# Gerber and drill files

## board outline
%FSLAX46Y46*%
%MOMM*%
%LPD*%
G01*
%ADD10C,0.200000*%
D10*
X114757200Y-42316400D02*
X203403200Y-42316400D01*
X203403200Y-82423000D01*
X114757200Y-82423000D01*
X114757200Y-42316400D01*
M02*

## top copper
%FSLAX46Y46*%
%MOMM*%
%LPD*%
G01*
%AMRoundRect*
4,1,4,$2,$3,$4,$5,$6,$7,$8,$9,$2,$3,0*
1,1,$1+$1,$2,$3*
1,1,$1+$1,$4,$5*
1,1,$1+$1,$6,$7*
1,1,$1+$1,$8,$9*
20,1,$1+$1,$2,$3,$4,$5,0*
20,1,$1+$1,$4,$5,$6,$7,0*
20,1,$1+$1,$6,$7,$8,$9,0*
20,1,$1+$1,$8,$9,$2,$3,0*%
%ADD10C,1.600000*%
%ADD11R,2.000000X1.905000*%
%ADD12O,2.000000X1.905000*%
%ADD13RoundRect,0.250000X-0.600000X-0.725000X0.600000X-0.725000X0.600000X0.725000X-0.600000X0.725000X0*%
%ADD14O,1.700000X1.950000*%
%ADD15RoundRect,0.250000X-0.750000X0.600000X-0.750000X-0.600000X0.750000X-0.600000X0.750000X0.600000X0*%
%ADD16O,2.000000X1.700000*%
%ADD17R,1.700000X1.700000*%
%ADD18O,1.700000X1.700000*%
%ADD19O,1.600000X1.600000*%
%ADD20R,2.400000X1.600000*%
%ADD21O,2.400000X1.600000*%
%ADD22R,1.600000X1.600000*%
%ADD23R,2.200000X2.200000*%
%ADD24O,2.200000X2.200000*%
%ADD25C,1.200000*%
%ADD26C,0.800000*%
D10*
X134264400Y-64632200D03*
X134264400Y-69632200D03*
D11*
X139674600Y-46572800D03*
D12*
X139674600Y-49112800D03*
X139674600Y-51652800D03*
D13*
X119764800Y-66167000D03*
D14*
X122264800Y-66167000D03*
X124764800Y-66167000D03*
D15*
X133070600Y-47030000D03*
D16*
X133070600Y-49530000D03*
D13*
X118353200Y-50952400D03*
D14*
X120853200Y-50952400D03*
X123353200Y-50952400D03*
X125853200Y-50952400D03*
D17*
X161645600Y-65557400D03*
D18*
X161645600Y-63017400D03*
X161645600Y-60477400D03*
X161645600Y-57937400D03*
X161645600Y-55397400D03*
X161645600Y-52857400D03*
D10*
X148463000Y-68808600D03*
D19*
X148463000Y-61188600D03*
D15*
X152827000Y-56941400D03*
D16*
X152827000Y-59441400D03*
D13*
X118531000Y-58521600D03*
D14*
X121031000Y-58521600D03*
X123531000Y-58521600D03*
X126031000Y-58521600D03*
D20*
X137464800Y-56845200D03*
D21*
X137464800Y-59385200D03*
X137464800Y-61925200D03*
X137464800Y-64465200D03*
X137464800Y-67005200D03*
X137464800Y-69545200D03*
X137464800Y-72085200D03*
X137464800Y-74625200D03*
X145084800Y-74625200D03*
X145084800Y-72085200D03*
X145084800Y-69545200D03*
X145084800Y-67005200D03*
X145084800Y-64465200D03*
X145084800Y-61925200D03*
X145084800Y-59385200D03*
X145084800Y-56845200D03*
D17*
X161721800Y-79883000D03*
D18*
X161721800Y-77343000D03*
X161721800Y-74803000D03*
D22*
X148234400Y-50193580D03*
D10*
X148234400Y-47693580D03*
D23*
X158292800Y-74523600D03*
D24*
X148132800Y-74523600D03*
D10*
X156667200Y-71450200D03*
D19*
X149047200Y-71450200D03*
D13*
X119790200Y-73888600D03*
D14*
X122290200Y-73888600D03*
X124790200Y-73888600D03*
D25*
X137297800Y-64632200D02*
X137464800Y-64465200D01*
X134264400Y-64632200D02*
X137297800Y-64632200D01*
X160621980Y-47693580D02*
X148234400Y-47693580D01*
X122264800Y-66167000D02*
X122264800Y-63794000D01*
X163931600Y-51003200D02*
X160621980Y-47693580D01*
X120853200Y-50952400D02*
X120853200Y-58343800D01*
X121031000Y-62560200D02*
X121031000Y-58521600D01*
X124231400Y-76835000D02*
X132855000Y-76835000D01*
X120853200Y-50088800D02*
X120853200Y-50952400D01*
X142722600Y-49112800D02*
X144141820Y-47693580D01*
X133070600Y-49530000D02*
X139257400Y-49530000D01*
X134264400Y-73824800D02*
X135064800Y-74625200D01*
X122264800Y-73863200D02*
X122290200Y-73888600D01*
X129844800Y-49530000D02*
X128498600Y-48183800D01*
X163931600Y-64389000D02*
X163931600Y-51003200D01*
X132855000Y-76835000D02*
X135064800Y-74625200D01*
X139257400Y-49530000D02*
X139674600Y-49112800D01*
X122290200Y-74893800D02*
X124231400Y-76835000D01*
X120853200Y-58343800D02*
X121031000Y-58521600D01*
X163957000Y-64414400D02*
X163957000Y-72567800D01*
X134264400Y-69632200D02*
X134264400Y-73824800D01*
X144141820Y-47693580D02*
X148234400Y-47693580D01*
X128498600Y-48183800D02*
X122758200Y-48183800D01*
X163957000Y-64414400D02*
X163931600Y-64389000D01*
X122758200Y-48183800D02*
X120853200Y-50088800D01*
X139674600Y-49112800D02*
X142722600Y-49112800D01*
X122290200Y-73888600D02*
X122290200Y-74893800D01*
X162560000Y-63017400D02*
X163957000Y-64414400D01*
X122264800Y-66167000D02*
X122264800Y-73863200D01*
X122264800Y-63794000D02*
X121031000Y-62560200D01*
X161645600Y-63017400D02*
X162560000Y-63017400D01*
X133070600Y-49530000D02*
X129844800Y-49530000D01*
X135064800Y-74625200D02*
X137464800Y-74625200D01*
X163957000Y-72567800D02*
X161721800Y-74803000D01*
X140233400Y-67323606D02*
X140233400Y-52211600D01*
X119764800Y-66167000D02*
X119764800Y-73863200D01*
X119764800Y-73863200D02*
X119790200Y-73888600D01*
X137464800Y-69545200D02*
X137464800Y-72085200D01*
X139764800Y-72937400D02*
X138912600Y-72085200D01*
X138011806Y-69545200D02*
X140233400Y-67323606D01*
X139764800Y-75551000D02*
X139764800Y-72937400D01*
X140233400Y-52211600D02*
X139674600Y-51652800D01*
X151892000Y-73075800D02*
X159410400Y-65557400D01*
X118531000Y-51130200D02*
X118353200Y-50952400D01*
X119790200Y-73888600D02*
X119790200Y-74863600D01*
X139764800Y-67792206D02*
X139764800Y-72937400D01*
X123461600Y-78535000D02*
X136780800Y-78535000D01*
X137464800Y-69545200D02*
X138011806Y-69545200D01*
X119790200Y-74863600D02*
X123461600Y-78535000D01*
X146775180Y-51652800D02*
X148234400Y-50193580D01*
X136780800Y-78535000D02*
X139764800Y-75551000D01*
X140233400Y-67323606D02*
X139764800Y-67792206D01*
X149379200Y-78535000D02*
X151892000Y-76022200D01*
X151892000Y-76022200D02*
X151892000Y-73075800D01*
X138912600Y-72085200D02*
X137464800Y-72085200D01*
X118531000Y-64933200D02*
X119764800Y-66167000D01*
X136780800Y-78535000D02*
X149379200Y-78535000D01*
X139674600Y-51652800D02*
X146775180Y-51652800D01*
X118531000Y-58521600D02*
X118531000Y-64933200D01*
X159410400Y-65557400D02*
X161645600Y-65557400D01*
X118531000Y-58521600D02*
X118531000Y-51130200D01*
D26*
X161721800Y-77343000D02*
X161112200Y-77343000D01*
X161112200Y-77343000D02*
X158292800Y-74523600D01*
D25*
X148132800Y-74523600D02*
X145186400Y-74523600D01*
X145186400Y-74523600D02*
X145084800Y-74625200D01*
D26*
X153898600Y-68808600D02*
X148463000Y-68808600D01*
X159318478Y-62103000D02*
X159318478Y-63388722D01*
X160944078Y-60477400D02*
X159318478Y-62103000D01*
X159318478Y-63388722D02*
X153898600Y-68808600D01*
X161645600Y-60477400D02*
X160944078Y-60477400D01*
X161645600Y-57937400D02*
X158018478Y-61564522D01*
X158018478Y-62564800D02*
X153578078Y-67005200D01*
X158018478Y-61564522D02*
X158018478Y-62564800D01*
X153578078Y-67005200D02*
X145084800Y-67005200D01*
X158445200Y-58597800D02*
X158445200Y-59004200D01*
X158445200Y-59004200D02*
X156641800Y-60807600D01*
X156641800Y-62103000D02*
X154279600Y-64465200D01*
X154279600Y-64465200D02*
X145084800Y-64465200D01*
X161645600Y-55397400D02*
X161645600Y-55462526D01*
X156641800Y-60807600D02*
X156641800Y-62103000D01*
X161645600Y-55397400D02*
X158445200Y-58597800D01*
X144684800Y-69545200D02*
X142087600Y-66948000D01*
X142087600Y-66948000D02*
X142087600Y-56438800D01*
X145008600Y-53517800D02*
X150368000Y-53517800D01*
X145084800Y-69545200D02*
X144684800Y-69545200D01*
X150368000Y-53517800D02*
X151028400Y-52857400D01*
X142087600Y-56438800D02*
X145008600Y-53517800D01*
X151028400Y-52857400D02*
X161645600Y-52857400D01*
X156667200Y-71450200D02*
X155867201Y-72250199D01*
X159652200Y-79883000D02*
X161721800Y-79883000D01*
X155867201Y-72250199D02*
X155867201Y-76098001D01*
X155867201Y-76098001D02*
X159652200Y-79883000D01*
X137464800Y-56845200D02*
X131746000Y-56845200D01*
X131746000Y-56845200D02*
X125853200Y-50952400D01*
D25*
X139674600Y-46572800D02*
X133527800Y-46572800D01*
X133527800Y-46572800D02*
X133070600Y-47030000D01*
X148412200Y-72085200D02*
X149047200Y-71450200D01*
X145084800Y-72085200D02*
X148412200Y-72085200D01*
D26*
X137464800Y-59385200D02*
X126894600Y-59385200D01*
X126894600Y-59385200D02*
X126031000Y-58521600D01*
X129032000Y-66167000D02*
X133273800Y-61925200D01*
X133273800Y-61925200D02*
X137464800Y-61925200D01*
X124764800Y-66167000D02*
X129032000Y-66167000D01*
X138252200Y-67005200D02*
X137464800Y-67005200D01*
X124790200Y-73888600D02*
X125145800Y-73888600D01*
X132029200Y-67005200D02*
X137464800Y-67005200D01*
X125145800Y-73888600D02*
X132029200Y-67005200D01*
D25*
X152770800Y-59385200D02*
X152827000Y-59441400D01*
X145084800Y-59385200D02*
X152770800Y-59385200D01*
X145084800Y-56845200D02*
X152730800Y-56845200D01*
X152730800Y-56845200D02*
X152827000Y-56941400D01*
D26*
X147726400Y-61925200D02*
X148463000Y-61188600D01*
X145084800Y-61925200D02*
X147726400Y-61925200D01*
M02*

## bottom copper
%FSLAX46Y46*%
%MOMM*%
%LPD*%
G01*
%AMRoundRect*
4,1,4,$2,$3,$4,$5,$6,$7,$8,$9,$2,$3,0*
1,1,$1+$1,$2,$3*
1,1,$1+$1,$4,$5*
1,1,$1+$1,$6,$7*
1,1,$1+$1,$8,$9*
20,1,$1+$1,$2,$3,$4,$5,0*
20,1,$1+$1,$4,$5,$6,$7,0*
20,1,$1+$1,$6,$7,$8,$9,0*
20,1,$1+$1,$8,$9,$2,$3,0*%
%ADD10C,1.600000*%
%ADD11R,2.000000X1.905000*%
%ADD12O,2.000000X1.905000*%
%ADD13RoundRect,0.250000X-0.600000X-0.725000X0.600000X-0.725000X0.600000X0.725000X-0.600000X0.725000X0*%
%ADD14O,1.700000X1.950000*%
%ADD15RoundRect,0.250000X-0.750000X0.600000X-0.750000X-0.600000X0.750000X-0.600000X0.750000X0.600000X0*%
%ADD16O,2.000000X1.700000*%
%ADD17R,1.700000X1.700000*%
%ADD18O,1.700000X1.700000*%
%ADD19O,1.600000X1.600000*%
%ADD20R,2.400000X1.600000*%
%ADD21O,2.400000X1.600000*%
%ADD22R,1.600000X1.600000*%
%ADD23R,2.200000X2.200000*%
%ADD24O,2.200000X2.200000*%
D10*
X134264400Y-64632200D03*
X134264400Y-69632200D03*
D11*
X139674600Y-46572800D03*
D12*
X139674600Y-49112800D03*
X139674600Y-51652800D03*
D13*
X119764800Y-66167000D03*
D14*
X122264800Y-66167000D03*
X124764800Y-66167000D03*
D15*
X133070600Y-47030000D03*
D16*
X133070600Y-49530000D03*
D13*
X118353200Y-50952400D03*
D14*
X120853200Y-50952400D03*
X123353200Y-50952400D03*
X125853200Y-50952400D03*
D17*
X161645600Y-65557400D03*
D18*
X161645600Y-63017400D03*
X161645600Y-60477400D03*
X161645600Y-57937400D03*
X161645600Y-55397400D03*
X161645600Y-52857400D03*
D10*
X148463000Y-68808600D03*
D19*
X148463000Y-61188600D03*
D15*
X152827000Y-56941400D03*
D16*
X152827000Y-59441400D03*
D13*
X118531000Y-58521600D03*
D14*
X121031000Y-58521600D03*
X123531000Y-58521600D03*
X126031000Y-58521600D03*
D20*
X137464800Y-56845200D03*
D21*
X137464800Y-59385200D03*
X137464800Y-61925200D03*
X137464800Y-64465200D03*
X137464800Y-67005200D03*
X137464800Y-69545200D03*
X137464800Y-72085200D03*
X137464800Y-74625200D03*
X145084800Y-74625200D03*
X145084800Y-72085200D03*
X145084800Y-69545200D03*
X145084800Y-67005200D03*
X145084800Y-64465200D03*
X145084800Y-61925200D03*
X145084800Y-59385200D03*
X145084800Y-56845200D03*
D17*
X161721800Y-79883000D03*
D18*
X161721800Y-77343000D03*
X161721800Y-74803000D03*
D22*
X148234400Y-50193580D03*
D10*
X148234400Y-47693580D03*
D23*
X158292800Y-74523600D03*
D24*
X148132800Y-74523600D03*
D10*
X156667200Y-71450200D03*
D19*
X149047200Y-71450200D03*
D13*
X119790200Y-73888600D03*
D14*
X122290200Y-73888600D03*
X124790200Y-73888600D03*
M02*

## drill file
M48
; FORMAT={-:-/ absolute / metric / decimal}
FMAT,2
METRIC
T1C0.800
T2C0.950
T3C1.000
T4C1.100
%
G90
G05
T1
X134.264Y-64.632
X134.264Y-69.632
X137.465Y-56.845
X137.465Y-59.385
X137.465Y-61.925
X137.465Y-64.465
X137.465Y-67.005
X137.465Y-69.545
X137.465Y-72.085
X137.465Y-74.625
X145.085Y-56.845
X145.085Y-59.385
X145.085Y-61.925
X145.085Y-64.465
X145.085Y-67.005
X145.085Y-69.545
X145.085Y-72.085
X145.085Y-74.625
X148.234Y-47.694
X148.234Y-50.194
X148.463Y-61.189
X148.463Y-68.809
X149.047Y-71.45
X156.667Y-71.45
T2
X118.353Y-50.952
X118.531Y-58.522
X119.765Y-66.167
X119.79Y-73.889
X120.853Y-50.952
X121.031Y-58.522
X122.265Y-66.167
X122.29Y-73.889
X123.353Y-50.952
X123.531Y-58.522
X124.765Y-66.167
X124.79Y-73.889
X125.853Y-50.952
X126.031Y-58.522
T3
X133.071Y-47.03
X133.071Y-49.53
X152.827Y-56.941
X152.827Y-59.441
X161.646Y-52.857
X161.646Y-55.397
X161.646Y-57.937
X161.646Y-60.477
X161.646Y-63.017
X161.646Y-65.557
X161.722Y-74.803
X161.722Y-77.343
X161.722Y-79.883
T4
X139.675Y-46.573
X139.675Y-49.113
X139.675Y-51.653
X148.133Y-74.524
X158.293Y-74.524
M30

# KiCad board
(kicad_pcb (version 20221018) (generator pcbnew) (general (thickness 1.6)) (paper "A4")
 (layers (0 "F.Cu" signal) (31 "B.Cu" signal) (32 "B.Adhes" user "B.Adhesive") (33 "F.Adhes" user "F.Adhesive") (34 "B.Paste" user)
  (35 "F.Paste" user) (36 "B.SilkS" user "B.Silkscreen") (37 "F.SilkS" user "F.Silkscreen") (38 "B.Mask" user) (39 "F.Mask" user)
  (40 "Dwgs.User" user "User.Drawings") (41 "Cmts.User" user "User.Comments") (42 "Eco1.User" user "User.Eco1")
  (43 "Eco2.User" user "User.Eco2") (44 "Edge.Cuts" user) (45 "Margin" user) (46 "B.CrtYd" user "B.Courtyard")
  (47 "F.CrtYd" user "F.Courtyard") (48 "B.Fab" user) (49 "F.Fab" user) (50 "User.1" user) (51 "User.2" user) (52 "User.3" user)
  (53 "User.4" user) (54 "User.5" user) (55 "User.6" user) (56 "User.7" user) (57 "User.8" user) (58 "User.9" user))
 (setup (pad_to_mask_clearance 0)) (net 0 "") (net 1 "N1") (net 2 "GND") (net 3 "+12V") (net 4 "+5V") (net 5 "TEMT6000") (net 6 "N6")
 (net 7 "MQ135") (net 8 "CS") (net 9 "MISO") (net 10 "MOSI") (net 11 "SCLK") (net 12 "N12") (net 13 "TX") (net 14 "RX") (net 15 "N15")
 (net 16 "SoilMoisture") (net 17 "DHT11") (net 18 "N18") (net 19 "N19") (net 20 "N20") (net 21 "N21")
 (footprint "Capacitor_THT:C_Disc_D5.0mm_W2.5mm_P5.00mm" (layer "F.Cu") (at 134.2644 64.6322 -90)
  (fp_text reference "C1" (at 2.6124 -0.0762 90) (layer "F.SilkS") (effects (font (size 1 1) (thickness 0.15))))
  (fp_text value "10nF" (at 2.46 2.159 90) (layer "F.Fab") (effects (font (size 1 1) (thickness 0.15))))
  (pad "1" thru_hole circle (at 0 0 270) (size 1.6 1.6) (drill 0.8) (layers "*.Cu" "*.Mask") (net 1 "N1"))
  (pad "2" thru_hole circle (at 5 0 270) (size 1.6 1.6) (drill 0.8) (layers "*.Cu" "*.Mask") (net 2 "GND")))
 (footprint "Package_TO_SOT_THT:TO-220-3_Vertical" (layer "F.Cu") (at 139.6746 46.5728 -90)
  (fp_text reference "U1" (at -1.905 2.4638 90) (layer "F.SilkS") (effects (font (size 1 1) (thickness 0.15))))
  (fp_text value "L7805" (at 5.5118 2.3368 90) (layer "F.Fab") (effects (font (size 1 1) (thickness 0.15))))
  (pad "1" thru_hole rect (at 0 0 270) (size 1.905 2) (drill 1.1) (layers "*.Cu" "*.Mask") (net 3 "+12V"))
  (pad "2" thru_hole oval (at 2.54 0 270) (size 1.905 2) (drill 1.1) (layers "*.Cu" "*.Mask") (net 2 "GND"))
  (pad "3" thru_hole oval (at 5.08 0 270) (size 1.905 2) (drill 1.1) (layers "*.Cu" "*.Mask") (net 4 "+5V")))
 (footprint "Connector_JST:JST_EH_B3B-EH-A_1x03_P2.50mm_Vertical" (layer "F.Cu") (at 119.7648 66.167)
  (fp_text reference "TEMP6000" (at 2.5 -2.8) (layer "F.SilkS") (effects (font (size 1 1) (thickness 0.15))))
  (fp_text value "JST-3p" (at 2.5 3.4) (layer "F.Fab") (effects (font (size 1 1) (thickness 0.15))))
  (pad "1" thru_hole roundrect (at 0 0) (size 1.7 1.95) (drill 0.95) (layers "*.Cu" "*.Mask") (roundrect_rratio 0.147059) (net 4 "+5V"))
  (pad "2" thru_hole oval (at 2.5 0) (size 1.7 1.95) (drill 0.95) (layers "*.Cu" "*.Mask") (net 2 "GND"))
  (pad "3" thru_hole oval (at 5 0) (size 1.7 1.95) (drill 0.95) (layers "*.Cu" "*.Mask") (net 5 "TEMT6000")))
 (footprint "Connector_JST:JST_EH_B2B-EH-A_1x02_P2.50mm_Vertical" (layer "F.Cu") (at 133.0706 47.03 -90)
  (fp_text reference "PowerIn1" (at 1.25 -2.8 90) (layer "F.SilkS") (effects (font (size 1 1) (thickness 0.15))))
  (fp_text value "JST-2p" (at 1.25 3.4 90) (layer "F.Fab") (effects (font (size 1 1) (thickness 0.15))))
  (pad "1" thru_hole roundrect (at 0 0 270) (size 1.7 2) (drill 1) (layers "*.Cu" "*.Mask") (roundrect_rratio 0.147059) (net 3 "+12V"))
  (pad "2" thru_hole oval (at 2.5 0 270) (size 1.7 2) (drill 1) (layers "*.Cu" "*.Mask") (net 2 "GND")))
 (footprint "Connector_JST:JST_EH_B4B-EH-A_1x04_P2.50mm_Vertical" (layer "F.Cu") (at 118.3532 50.9524)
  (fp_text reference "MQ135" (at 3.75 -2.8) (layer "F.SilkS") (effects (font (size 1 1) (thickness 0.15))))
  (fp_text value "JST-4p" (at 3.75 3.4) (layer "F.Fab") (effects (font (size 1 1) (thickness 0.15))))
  (pad "1" thru_hole roundrect (at 0 0) (size 1.7 1.95) (drill 0.95) (layers "*.Cu" "*.Mask") (roundrect_rratio 0.147059) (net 4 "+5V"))
  (pad "2" thru_hole oval (at 2.5 0) (size 1.7 1.95) (drill 0.95) (layers "*.Cu" "*.Mask") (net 2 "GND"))
  (pad "3" thru_hole oval (at 5 0) (size 1.7 1.95) (drill 0.95) (layers "*.Cu" "*.Mask") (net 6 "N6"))
  (pad "4" thru_hole oval (at 7.5 0) (size 1.7 1.95) (drill 0.95) (layers "*.Cu" "*.Mask") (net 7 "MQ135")))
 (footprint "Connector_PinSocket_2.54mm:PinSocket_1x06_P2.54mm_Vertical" (layer "F.Cu") (at 161.6456 65.5574 180)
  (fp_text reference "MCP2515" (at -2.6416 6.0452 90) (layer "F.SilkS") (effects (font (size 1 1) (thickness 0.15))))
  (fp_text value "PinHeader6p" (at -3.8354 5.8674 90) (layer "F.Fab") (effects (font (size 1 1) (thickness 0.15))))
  (pad "1" thru_hole rect (at 0 0 180) (size 1.7 1.7) (drill 1) (layers "*.Cu" "*.Mask") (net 4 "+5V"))
  (pad "2" thru_hole oval (at 0 2.54 180) (size 1.7 1.7) (drill 1) (layers "*.Cu" "*.Mask") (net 2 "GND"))
  (pad "3" thru_hole oval (at 0 5.08 180) (size 1.7 1.7) (drill 1) (layers "*.Cu" "*.Mask") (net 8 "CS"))
  (pad "4" thru_hole oval (at 0 7.62 180) (size 1.7 1.7) (drill 1) (layers "*.Cu" "*.Mask") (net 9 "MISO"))
  (pad "5" thru_hole oval (at 0 10.16 180) (size 1.7 1.7) (drill 1) (layers "*.Cu" "*.Mask") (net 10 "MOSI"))
  (pad "6" thru_hole oval (at 0 12.7 180) (size 1.7 1.7) (drill 1) (layers "*.Cu" "*.Mask") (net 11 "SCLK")))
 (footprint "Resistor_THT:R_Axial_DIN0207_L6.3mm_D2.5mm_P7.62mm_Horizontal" (layer "F.Cu") (at 148.463 68.8086 90)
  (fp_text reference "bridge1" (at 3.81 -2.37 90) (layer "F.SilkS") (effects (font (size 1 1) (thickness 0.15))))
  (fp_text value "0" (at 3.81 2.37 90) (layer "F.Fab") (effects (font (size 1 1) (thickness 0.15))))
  (pad "1" thru_hole circle (at 0 0 90) (size 1.6 1.6) (drill 0.8) (layers "*.Cu" "*.Mask") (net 8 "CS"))
  (pad "2" thru_hole oval (at 7.62 0 90) (size 1.6 1.6) (drill 0.8) (layers "*.Cu" "*.Mask") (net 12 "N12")))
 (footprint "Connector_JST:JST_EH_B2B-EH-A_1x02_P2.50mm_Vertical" (layer "F.Cu") (at 152.827 56.9414 -90)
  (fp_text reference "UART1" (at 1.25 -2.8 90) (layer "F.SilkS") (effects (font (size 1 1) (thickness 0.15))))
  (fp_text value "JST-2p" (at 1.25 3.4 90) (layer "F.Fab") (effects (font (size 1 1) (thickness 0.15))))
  (pad "1" thru_hole roundrect (at 0 0 270) (size 1.7 2) (drill 1) (layers "*.Cu" "*.Mask") (roundrect_rratio 0.147059) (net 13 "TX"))
  (pad "2" thru_hole oval (at 2.5 0 270) (size 1.7 2) (drill 1) (layers "*.Cu" "*.Mask") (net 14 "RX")))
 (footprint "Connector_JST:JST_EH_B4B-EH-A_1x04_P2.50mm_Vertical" (layer "F.Cu") (at 118.531 58.5216)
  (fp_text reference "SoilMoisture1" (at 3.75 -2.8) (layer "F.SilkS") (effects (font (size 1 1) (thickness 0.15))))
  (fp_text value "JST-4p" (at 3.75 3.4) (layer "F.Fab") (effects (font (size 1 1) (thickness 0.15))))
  (pad "1" thru_hole roundrect (at 0 0) (size 1.7 1.95) (drill 0.95) (layers "*.Cu" "*.Mask") (roundrect_rratio 0.147059) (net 4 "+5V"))
  (pad "2" thru_hole oval (at 2.5 0) (size 1.7 1.95) (drill 0.95) (layers "*.Cu" "*.Mask") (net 2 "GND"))
  (pad "3" thru_hole oval (at 5 0) (size 1.7 1.95) (drill 0.95) (layers "*.Cu" "*.Mask") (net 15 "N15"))
  (pad "4" thru_hole oval (at 7.5 0) (size 1.7 1.95) (drill 0.95) (layers "*.Cu" "*.Mask") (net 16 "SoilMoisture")))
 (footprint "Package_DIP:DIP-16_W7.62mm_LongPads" (layer "F.Cu") (at 137.4648 56.8452)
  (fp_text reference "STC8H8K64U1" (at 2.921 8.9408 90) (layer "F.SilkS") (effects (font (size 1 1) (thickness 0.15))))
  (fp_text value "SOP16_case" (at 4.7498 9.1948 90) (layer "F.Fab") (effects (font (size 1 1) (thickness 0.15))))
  (pad "1" thru_hole rect (at 0 0) (size 2.4 1.6) (drill 0.8) (layers "*.Cu" "*.Mask") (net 7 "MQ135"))
  (pad "2" thru_hole oval (at 0 2.54) (size 2.4 1.6) (drill 0.8) (layers "*.Cu" "*.Mask") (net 16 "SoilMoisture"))
  (pad "3" thru_hole oval (at 0 5.08) (size 2.4 1.6) (drill 0.8) (layers "*.Cu" "*.Mask") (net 5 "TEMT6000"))
  (pad "4" thru_hole oval (at 0 7.62) (size 2.4 1.6) (drill 0.8) (layers "*.Cu" "*.Mask") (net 1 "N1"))
  (pad "5" thru_hole oval (at 0 10.16) (size 2.4 1.6) (drill 0.8) (layers "*.Cu" "*.Mask") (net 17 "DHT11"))
  (pad "6" thru_hole oval (at 0 12.7) (size 2.4 1.6) (drill 0.8) (layers "*.Cu" "*.Mask") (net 4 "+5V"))
  (pad "7" thru_hole oval (at 0 15.24) (size 2.4 1.6) (drill 0.8) (layers "*.Cu" "*.Mask") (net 4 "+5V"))
  (pad "8" thru_hole oval (at 0 17.78) (size 2.4 1.6) (drill 0.8) (layers "*.Cu" "*.Mask") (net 2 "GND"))
  (pad "9" thru_hole oval (at 7.62 17.78) (size 2.4 1.6) (drill 0.8) (layers "*.Cu" "*.Mask") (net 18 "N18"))
  (pad "10" thru_hole oval (at 7.62 15.24) (size 2.4 1.6) (drill 0.8) (layers "*.Cu" "*.Mask") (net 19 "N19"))
  (pad "11" thru_hole oval (at 7.62 12.7) (size 2.4 1.6) (drill 0.8) (layers "*.Cu" "*.Mask") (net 11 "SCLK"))
  (pad "12" thru_hole oval (at 7.62 10.16) (size 2.4 1.6) (drill 0.8) (layers "*.Cu" "*.Mask") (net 9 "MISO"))
  (pad "13" thru_hole oval (at 7.62 7.62) (size 2.4 1.6) (drill 0.8) (layers "*.Cu" "*.Mask") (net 10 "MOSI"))
  (pad "14" thru_hole oval (at 7.62 5.08) (size 2.4 1.6) (drill 0.8) (layers "*.Cu" "*.Mask") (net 12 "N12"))
  (pad "15" thru_hole oval (at 7.62 2.54) (size 2.4 1.6) (drill 0.8) (layers "*.Cu" "*.Mask") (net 14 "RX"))
  (pad "16" thru_hole oval (at 7.62 0) (size 2.4 1.6) (drill 0.8) (layers "*.Cu" "*.Mask") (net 13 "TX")))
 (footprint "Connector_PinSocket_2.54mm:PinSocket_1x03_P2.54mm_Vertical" (layer "F.Cu") (at 161.7218 79.883 180)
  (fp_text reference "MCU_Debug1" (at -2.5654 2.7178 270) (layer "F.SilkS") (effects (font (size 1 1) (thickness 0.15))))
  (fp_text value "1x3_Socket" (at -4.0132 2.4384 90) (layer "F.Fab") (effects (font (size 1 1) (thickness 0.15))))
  (pad "1" thru_hole rect (at 0 0 180) (size 1.7 1.7) (drill 1) (layers "*.Cu" "*.Mask") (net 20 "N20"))
  (pad "2" thru_hole oval (at 0 2.54 180) (size 1.7 1.7) (drill 1) (layers "*.Cu" "*.Mask") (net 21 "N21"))
  (pad "3" thru_hole oval (at 0 5.08 180) (size 1.7 1.7) (drill 1) (layers "*.Cu" "*.Mask") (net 2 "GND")))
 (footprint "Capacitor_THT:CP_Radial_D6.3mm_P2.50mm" (layer "F.Cu") (at 148.2344 50.19358 90)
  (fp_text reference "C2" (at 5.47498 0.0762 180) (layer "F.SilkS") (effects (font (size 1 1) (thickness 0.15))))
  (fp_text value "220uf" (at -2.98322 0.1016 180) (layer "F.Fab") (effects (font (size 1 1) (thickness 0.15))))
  (pad "1" thru_hole rect (at 0 0 90) (size 1.6 1.6) (drill 0.8) (layers "*.Cu" "*.Mask") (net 4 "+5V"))
  (pad "2" thru_hole circle (at 2.5 0 90) (size 1.6 1.6) (drill 0.8) (layers "*.Cu" "*.Mask") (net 2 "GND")))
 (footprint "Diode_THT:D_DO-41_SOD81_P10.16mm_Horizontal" (layer "F.Cu") (at 158.2928 74.5236 180)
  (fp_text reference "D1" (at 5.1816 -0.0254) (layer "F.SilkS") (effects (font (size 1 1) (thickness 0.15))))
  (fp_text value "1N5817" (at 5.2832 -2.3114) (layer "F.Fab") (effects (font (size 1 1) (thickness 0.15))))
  (pad "1" thru_hole rect (at 0 0 180) (size 2.2 2.2) (drill 1.1) (layers "*.Cu" "*.Mask") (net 21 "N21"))
  (pad "2" thru_hole oval (at 10.16 0 180) (size 2.2 2.2) (drill 1.1) (layers "*.Cu" "*.Mask") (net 18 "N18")))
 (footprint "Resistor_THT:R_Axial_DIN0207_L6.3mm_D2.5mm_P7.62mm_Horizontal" (layer "F.Cu") (at 156.6672 71.4502 180)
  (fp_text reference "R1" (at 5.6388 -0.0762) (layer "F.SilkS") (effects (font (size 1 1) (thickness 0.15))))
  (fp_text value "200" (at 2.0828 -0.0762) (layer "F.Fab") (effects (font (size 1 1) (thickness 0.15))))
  (pad "1" thru_hole circle (at 0 0 180) (size 1.6 1.6) (drill 0.8) (layers "*.Cu" "*.Mask") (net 20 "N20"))
  (pad "2" thru_hole oval (at 7.62 0 180) (size 1.6 1.6) (drill 0.8) (layers "*.Cu" "*.Mask") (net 19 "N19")))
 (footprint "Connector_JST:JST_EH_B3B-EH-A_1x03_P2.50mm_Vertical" (layer "F.Cu") (at 119.7902 73.8886)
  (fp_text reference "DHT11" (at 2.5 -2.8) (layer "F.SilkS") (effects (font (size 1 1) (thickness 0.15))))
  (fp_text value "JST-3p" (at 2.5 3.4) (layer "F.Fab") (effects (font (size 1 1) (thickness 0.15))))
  (pad "1" thru_hole roundrect (at 0 0) (size 1.7 1.95) (drill 0.95) (layers "*.Cu" "*.Mask") (roundrect_rratio 0.147059) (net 4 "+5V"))
  (pad "2" thru_hole oval (at 2.5 0) (size 1.7 1.95) (drill 0.95) (layers "*.Cu" "*.Mask") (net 2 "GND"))
  (pad "3" thru_hole oval (at 5 0) (size 1.7 1.95) (drill 0.95) (layers "*.Cu" "*.Mask") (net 17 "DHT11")))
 (gr_rect (start 114.7572 42.3164) (end 203.4032 82.423) (stroke (width 0.2) (type default)) (fill none) (layer "Edge.Cuts"))
 (segment (start 137.2978 64.6322) (end 137.4648 64.4652) (width 1.2) (layer "F.Cu") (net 1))
 (segment (start 134.2644 64.6322) (end 137.2978 64.6322) (width 1.2) (layer "F.Cu") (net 1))
 (segment (start 160.62198 47.69358) (end 148.2344 47.69358) (width 1.2) (layer "F.Cu") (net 2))
 (segment (start 122.2648 66.167) (end 122.2648 63.794) (width 1.2) (layer "F.Cu") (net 2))
 (segment (start 163.9316 51.0032) (end 160.62198 47.69358) (width 1.2) (layer "F.Cu") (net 2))
 (segment (start 120.8532 50.9524) (end 120.8532 58.3438) (width 1.2) (layer "F.Cu") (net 2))
 (segment (start 121.031 62.5602) (end 121.031 58.5216) (width 1.2) (layer "F.Cu") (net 2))
 (segment (start 124.2314 76.835) (end 132.855 76.835) (width 1.2) (layer "F.Cu") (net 2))
 (segment (start 120.8532 50.0888) (end 120.8532 50.9524) (width 1.2) (layer "F.Cu") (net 2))
 (segment (start 142.7226 49.1128) (end 144.14182 47.69358) (width 1.2) (layer "F.Cu") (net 2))
 (segment (start 133.0706 49.53) (end 139.2574 49.53) (width 1.2) (layer "F.Cu") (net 2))
 (segment (start 134.2644 73.8248) (end 135.0648 74.6252) (width 1.2) (layer "F.Cu") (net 2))
 (segment (start 122.2648 73.8632) (end 122.2902 73.8886) (width 1.2) (layer "F.Cu") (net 2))
 (segment (start 129.8448 49.53) (end 128.4986 48.1838) (width 1.2) (layer "F.Cu") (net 2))
 (segment (start 163.9316 64.389) (end 163.9316 51.0032) (width 1.2) (layer "F.Cu") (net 2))
 (segment (start 132.855 76.835) (end 135.0648 74.6252) (width 1.2) (layer "F.Cu") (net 2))
 (segment (start 139.2574 49.53) (end 139.6746 49.1128) (width 1.2) (layer "F.Cu") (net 2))
 (segment (start 122.2902 74.8938) (end 124.2314 76.835) (width 1.2) (layer "F.Cu") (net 2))
 (segment (start 120.8532 58.3438) (end 121.031 58.5216) (width 1.2) (layer "F.Cu") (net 2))
 (segment (start 163.957 64.4144) (end 163.957 72.5678) (width 1.2) (layer "F.Cu") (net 2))
 (segment (start 134.2644 69.6322) (end 134.2644 73.8248) (width 1.2) (layer "F.Cu") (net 2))
 (segment (start 144.14182 47.69358) (end 148.2344 47.69358) (width 1.2) (layer "F.Cu") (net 2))
 (segment (start 128.4986 48.1838) (end 122.7582 48.1838) (width 1.2) (layer "F.Cu") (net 2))
 (segment (start 163.957 64.4144) (end 163.9316 64.389) (width 1.2) (layer "F.Cu") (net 2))
 (segment (start 122.7582 48.1838) (end 120.8532 50.0888) (width 1.2) (layer "F.Cu") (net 2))
 (segment (start 139.6746 49.1128) (end 142.7226 49.1128) (width 1.2) (layer "F.Cu") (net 2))
 (segment (start 122.2902 73.8886) (end 122.2902 74.8938) (width 1.2) (layer "F.Cu") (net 2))
 (segment (start 162.56 63.0174) (end 163.957 64.4144) (width 1.2) (layer "F.Cu") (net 2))
 (segment (start 122.2648 66.167) (end 122.2648 73.8632) (width 1.2) (layer "F.Cu") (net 2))
 (segment (start 122.2648 63.794) (end 121.031 62.5602) (width 1.2) (layer "F.Cu") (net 2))
 (segment (start 161.6456 63.0174) (end 162.56 63.0174) (width 1.2) (layer "F.Cu") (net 2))
 (segment (start 133.0706 49.53) (end 129.8448 49.53) (width 1.2) (layer "F.Cu") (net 2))
 (segment (start 135.0648 74.6252) (end 137.4648 74.6252) (width 1.2) (layer "F.Cu") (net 2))
 (segment (start 163.957 72.5678) (end 161.7218 74.803) (width 1.2) (layer "F.Cu") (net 2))
 (segment (start 140.2334 67.323606) (end 140.2334 52.2116) (width 1.2) (layer "F.Cu") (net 4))
 (segment (start 119.7648 66.167) (end 119.7648 73.8632) (width 1.2) (layer "F.Cu") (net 4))
 (segment (start 119.7648 73.8632) (end 119.7902 73.8886) (width 1.2) (layer "F.Cu") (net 4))
 (segment (start 137.4648 69.5452) (end 137.4648 72.0852) (width 1.2) (layer "F.Cu") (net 4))
 (segment (start 139.7648 72.9374) (end 138.9126 72.0852) (width 1.2) (layer "F.Cu") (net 4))
 (segment (start 138.011806 69.5452) (end 140.2334 67.323606) (width 1.2) (layer "F.Cu") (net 4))
 (segment (start 139.7648 75.551) (end 139.7648 72.9374) (width 1.2) (layer "F.Cu") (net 4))
 (segment (start 140.2334 52.2116) (end 139.6746 51.6528) (width 1.2) (layer "F.Cu") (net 4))
 (segment (start 151.892 73.0758) (end 159.4104 65.5574) (width 1.2) (layer "F.Cu") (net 4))
 (segment (start 118.531 51.1302) (end 118.3532 50.9524) (width 1.2) (layer "F.Cu") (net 4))
 (segment (start 119.7902 73.8886) (end 119.7902 74.8636) (width 1.2) (layer "F.Cu") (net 4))
 (segment (start 139.7648 67.792206) (end 139.7648 72.9374) (width 1.2) (layer "F.Cu") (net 4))
 (segment (start 123.4616 78.535) (end 136.7808 78.535) (width 1.2) (layer "F.Cu") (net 4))
 (segment (start 137.4648 69.5452) (end 138.011806 69.5452) (width 1.2) (layer "F.Cu") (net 4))
 (segment (start 119.7902 74.8636) (end 123.4616 78.535) (width 1.2) (layer "F.Cu") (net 4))
 (segment (start 146.77518 51.6528) (end 148.2344 50.19358) (width 1.2) (layer "F.Cu") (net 4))
 (segment (start 136.7808 78.535) (end 139.7648 75.551) (width 1.2) (layer "F.Cu") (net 4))
 (segment (start 140.2334 67.323606) (end 139.7648 67.792206) (width 1.2) (layer "F.Cu") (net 4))
 (segment (start 149.3792 78.535) (end 151.892 76.0222) (width 1.2) (layer "F.Cu") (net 4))
 (segment (start 151.892 76.0222) (end 151.892 73.0758) (width 1.2) (layer "F.Cu") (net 4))
 (segment (start 138.9126 72.0852) (end 137.4648 72.0852) (width 1.2) (layer "F.Cu") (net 4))
 (segment (start 118.531 64.9332) (end 119.7648 66.167) (width 1.2) (layer "F.Cu") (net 4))
 (segment (start 136.7808 78.535) (end 149.3792 78.535) (width 1.2) (layer "F.Cu") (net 4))
 (segment (start 139.6746 51.6528) (end 146.77518 51.6528) (width 1.2) (layer "F.Cu") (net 4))
 (segment (start 118.531 58.5216) (end 118.531 64.9332) (width 1.2) (layer "F.Cu") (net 4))
 (segment (start 159.4104 65.5574) (end 161.6456 65.5574) (width 1.2) (layer "F.Cu") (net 4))
 (segment (start 118.531 58.5216) (end 118.531 51.1302) (width 1.2) (layer "F.Cu") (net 4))
 (segment (start 161.7218 77.343) (end 161.1122 77.343) (width 0.8) (layer "F.Cu") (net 21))
 (segment (start 161.1122 77.343) (end 158.2928 74.5236) (width 0.8) (layer "F.Cu") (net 21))
 (segment (start 148.1328 74.5236) (end 145.1864 74.5236) (width 1.2) (layer "F.Cu") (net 18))
 (segment (start 145.1864 74.5236) (end 145.0848 74.6252) (width 1.2) (layer "F.Cu") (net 18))
 (segment (start 153.8986 68.8086) (end 148.463 68.8086) (width 0.8) (layer "F.Cu") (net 8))
 (segment (start 159.318478 62.103) (end 159.318478 63.388722) (width 0.8) (layer "F.Cu") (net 8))
 (segment (start 160.944078 60.4774) (end 159.318478 62.103) (width 0.8) (layer "F.Cu") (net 8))
 (segment (start 159.318478 63.388722) (end 153.8986 68.8086) (width 0.8) (layer "F.Cu") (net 8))
 (segment (start 161.6456 60.4774) (end 160.944078 60.4774) (width 0.8) (layer "F.Cu") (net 8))
 (segment (start 161.6456 57.9374) (end 158.018478 61.564522) (width 0.8) (layer "F.Cu") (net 9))
 (segment (start 158.018478 62.5648) (end 153.578078 67.0052) (width 0.8) (layer "F.Cu") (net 9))
 (segment (start 158.018478 61.564522) (end 158.018478 62.5648) (width 0.8) (layer "F.Cu") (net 9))
 (segment (start 153.578078 67.0052) (end 145.0848 67.0052) (width 0.8) (layer "F.Cu") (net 9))
 (segment (start 158.4452 58.5978) (end 158.4452 59.0042) (width 0.8) (layer "F.Cu") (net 10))
 (segment (start 158.4452 59.0042) (end 156.6418 60.8076) (width 0.8) (layer "F.Cu") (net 10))
 (segment (start 156.6418 62.103) (end 154.2796 64.4652) (width 0.8) (layer "F.Cu") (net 10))
 (segment (start 154.2796 64.4652) (end 145.0848 64.4652) (width 0.8) (layer "F.Cu") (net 10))
 (segment (start 161.6456 55.3974) (end 161.6456 55.462526) (width 0.8) (layer "F.Cu") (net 10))
 (segment (start 156.6418 60.8076) (end 156.6418 62.103) (width 0.8) (layer "F.Cu") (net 10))
 (segment (start 161.6456 55.3974) (end 158.4452 58.5978) (width 0.8) (layer "F.Cu") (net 10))
 (segment (start 144.6848 69.5452) (end 142.0876 66.948) (width 0.8) (layer "F.Cu") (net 11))
 (segment (start 142.0876 66.948) (end 142.0876 56.4388) (width 0.8) (layer "F.Cu") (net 11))
 (segment (start 145.0086 53.5178) (end 150.368 53.5178) (width 0.8) (layer "F.Cu") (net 11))
 (segment (start 145.0848 69.5452) (end 144.6848 69.5452) (width 0.8) (layer "F.Cu") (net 11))
 (segment (start 150.368 53.5178) (end 151.0284 52.8574) (width 0.8) (layer "F.Cu") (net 11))
 (segment (start 142.0876 56.4388) (end 145.0086 53.5178) (width 0.8) (layer "F.Cu") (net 11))
 (segment (start 151.0284 52.8574) (end 161.6456 52.8574) (width 0.8) (layer "F.Cu") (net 11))
 (segment (start 156.6672 71.4502) (end 155.867201 72.250199) (width 0.8) (layer "F.Cu") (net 20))
 (segment (start 159.6522 79.883) (end 161.7218 79.883) (width 0.8) (layer "F.Cu") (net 20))
 (segment (start 155.867201 72.250199) (end 155.867201 76.098001) (width 0.8) (layer "F.Cu") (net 20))
 (segment (start 155.867201 76.098001) (end 159.6522 79.883) (width 0.8) (layer "F.Cu") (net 20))
 (segment (start 137.4648 56.8452) (end 131.746 56.8452) (width 0.8) (layer "F.Cu") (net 7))
 (segment (start 131.746 56.8452) (end 125.8532 50.9524) (width 0.8) (layer "F.Cu") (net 7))
 (segment (start 139.6746 46.5728) (end 133.5278 46.5728) (width 1.2) (layer "F.Cu") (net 3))
 (segment (start 133.5278 46.5728) (end 133.0706 47.03) (width 1.2) (layer "F.Cu") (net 3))
 (segment (start 148.4122 72.0852) (end 149.0472 71.4502) (width 1.2) (layer "F.Cu") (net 19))
 (segment (start 145.0848 72.0852) (end 148.4122 72.0852) (width 1.2) (layer "F.Cu") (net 19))
 (segment (start 137.4648 59.3852) (end 126.8946 59.3852) (width 0.8) (layer "F.Cu") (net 16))
 (segment (start 126.8946 59.3852) (end 126.031 58.5216) (width 0.8) (layer "F.Cu") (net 16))
 (segment (start 129.032 66.167) (end 133.2738 61.9252) (width 0.8) (layer "F.Cu") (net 5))
 (segment (start 133.2738 61.9252) (end 137.4648 61.9252) (width 0.8) (layer "F.Cu") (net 5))
 (segment (start 124.7648 66.167) (end 129.032 66.167) (width 0.8) (layer "F.Cu") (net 5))
 (segment (start 138.2522 67.0052) (end 137.4648 67.0052) (width 0.8) (layer "F.Cu") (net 17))
 (segment (start 124.7902 73.8886) (end 125.1458 73.8886) (width 0.8) (layer "F.Cu") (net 17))
 (segment (start 132.0292 67.0052) (end 137.4648 67.0052) (width 0.8) (layer "F.Cu") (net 17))
 (segment (start 125.1458 73.8886) (end 132.0292 67.0052) (width 0.8) (layer "F.Cu") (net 17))
 (segment (start 152.7708 59.3852) (end 152.827 59.4414) (width 1.2) (layer "F.Cu") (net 14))
 (segment (start 145.0848 59.3852) (end 152.7708 59.3852) (width 1.2) (layer "F.Cu") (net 14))
 (segment (start 145.0848 56.8452) (end 152.7308 56.8452) (width 1.2) (layer "F.Cu") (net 13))
 (segment (start 152.7308 56.8452) (end 152.827 56.9414) (width 1.2) (layer "F.Cu") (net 13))
 (segment (start 147.7264 61.9252) (end 148.463 61.1886) (width 0.8) (layer "F.Cu") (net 12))
 (segment (start 145.0848 61.9252) (end 147.7264 61.9252) (width 0.8) (layer "F.Cu") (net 12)))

